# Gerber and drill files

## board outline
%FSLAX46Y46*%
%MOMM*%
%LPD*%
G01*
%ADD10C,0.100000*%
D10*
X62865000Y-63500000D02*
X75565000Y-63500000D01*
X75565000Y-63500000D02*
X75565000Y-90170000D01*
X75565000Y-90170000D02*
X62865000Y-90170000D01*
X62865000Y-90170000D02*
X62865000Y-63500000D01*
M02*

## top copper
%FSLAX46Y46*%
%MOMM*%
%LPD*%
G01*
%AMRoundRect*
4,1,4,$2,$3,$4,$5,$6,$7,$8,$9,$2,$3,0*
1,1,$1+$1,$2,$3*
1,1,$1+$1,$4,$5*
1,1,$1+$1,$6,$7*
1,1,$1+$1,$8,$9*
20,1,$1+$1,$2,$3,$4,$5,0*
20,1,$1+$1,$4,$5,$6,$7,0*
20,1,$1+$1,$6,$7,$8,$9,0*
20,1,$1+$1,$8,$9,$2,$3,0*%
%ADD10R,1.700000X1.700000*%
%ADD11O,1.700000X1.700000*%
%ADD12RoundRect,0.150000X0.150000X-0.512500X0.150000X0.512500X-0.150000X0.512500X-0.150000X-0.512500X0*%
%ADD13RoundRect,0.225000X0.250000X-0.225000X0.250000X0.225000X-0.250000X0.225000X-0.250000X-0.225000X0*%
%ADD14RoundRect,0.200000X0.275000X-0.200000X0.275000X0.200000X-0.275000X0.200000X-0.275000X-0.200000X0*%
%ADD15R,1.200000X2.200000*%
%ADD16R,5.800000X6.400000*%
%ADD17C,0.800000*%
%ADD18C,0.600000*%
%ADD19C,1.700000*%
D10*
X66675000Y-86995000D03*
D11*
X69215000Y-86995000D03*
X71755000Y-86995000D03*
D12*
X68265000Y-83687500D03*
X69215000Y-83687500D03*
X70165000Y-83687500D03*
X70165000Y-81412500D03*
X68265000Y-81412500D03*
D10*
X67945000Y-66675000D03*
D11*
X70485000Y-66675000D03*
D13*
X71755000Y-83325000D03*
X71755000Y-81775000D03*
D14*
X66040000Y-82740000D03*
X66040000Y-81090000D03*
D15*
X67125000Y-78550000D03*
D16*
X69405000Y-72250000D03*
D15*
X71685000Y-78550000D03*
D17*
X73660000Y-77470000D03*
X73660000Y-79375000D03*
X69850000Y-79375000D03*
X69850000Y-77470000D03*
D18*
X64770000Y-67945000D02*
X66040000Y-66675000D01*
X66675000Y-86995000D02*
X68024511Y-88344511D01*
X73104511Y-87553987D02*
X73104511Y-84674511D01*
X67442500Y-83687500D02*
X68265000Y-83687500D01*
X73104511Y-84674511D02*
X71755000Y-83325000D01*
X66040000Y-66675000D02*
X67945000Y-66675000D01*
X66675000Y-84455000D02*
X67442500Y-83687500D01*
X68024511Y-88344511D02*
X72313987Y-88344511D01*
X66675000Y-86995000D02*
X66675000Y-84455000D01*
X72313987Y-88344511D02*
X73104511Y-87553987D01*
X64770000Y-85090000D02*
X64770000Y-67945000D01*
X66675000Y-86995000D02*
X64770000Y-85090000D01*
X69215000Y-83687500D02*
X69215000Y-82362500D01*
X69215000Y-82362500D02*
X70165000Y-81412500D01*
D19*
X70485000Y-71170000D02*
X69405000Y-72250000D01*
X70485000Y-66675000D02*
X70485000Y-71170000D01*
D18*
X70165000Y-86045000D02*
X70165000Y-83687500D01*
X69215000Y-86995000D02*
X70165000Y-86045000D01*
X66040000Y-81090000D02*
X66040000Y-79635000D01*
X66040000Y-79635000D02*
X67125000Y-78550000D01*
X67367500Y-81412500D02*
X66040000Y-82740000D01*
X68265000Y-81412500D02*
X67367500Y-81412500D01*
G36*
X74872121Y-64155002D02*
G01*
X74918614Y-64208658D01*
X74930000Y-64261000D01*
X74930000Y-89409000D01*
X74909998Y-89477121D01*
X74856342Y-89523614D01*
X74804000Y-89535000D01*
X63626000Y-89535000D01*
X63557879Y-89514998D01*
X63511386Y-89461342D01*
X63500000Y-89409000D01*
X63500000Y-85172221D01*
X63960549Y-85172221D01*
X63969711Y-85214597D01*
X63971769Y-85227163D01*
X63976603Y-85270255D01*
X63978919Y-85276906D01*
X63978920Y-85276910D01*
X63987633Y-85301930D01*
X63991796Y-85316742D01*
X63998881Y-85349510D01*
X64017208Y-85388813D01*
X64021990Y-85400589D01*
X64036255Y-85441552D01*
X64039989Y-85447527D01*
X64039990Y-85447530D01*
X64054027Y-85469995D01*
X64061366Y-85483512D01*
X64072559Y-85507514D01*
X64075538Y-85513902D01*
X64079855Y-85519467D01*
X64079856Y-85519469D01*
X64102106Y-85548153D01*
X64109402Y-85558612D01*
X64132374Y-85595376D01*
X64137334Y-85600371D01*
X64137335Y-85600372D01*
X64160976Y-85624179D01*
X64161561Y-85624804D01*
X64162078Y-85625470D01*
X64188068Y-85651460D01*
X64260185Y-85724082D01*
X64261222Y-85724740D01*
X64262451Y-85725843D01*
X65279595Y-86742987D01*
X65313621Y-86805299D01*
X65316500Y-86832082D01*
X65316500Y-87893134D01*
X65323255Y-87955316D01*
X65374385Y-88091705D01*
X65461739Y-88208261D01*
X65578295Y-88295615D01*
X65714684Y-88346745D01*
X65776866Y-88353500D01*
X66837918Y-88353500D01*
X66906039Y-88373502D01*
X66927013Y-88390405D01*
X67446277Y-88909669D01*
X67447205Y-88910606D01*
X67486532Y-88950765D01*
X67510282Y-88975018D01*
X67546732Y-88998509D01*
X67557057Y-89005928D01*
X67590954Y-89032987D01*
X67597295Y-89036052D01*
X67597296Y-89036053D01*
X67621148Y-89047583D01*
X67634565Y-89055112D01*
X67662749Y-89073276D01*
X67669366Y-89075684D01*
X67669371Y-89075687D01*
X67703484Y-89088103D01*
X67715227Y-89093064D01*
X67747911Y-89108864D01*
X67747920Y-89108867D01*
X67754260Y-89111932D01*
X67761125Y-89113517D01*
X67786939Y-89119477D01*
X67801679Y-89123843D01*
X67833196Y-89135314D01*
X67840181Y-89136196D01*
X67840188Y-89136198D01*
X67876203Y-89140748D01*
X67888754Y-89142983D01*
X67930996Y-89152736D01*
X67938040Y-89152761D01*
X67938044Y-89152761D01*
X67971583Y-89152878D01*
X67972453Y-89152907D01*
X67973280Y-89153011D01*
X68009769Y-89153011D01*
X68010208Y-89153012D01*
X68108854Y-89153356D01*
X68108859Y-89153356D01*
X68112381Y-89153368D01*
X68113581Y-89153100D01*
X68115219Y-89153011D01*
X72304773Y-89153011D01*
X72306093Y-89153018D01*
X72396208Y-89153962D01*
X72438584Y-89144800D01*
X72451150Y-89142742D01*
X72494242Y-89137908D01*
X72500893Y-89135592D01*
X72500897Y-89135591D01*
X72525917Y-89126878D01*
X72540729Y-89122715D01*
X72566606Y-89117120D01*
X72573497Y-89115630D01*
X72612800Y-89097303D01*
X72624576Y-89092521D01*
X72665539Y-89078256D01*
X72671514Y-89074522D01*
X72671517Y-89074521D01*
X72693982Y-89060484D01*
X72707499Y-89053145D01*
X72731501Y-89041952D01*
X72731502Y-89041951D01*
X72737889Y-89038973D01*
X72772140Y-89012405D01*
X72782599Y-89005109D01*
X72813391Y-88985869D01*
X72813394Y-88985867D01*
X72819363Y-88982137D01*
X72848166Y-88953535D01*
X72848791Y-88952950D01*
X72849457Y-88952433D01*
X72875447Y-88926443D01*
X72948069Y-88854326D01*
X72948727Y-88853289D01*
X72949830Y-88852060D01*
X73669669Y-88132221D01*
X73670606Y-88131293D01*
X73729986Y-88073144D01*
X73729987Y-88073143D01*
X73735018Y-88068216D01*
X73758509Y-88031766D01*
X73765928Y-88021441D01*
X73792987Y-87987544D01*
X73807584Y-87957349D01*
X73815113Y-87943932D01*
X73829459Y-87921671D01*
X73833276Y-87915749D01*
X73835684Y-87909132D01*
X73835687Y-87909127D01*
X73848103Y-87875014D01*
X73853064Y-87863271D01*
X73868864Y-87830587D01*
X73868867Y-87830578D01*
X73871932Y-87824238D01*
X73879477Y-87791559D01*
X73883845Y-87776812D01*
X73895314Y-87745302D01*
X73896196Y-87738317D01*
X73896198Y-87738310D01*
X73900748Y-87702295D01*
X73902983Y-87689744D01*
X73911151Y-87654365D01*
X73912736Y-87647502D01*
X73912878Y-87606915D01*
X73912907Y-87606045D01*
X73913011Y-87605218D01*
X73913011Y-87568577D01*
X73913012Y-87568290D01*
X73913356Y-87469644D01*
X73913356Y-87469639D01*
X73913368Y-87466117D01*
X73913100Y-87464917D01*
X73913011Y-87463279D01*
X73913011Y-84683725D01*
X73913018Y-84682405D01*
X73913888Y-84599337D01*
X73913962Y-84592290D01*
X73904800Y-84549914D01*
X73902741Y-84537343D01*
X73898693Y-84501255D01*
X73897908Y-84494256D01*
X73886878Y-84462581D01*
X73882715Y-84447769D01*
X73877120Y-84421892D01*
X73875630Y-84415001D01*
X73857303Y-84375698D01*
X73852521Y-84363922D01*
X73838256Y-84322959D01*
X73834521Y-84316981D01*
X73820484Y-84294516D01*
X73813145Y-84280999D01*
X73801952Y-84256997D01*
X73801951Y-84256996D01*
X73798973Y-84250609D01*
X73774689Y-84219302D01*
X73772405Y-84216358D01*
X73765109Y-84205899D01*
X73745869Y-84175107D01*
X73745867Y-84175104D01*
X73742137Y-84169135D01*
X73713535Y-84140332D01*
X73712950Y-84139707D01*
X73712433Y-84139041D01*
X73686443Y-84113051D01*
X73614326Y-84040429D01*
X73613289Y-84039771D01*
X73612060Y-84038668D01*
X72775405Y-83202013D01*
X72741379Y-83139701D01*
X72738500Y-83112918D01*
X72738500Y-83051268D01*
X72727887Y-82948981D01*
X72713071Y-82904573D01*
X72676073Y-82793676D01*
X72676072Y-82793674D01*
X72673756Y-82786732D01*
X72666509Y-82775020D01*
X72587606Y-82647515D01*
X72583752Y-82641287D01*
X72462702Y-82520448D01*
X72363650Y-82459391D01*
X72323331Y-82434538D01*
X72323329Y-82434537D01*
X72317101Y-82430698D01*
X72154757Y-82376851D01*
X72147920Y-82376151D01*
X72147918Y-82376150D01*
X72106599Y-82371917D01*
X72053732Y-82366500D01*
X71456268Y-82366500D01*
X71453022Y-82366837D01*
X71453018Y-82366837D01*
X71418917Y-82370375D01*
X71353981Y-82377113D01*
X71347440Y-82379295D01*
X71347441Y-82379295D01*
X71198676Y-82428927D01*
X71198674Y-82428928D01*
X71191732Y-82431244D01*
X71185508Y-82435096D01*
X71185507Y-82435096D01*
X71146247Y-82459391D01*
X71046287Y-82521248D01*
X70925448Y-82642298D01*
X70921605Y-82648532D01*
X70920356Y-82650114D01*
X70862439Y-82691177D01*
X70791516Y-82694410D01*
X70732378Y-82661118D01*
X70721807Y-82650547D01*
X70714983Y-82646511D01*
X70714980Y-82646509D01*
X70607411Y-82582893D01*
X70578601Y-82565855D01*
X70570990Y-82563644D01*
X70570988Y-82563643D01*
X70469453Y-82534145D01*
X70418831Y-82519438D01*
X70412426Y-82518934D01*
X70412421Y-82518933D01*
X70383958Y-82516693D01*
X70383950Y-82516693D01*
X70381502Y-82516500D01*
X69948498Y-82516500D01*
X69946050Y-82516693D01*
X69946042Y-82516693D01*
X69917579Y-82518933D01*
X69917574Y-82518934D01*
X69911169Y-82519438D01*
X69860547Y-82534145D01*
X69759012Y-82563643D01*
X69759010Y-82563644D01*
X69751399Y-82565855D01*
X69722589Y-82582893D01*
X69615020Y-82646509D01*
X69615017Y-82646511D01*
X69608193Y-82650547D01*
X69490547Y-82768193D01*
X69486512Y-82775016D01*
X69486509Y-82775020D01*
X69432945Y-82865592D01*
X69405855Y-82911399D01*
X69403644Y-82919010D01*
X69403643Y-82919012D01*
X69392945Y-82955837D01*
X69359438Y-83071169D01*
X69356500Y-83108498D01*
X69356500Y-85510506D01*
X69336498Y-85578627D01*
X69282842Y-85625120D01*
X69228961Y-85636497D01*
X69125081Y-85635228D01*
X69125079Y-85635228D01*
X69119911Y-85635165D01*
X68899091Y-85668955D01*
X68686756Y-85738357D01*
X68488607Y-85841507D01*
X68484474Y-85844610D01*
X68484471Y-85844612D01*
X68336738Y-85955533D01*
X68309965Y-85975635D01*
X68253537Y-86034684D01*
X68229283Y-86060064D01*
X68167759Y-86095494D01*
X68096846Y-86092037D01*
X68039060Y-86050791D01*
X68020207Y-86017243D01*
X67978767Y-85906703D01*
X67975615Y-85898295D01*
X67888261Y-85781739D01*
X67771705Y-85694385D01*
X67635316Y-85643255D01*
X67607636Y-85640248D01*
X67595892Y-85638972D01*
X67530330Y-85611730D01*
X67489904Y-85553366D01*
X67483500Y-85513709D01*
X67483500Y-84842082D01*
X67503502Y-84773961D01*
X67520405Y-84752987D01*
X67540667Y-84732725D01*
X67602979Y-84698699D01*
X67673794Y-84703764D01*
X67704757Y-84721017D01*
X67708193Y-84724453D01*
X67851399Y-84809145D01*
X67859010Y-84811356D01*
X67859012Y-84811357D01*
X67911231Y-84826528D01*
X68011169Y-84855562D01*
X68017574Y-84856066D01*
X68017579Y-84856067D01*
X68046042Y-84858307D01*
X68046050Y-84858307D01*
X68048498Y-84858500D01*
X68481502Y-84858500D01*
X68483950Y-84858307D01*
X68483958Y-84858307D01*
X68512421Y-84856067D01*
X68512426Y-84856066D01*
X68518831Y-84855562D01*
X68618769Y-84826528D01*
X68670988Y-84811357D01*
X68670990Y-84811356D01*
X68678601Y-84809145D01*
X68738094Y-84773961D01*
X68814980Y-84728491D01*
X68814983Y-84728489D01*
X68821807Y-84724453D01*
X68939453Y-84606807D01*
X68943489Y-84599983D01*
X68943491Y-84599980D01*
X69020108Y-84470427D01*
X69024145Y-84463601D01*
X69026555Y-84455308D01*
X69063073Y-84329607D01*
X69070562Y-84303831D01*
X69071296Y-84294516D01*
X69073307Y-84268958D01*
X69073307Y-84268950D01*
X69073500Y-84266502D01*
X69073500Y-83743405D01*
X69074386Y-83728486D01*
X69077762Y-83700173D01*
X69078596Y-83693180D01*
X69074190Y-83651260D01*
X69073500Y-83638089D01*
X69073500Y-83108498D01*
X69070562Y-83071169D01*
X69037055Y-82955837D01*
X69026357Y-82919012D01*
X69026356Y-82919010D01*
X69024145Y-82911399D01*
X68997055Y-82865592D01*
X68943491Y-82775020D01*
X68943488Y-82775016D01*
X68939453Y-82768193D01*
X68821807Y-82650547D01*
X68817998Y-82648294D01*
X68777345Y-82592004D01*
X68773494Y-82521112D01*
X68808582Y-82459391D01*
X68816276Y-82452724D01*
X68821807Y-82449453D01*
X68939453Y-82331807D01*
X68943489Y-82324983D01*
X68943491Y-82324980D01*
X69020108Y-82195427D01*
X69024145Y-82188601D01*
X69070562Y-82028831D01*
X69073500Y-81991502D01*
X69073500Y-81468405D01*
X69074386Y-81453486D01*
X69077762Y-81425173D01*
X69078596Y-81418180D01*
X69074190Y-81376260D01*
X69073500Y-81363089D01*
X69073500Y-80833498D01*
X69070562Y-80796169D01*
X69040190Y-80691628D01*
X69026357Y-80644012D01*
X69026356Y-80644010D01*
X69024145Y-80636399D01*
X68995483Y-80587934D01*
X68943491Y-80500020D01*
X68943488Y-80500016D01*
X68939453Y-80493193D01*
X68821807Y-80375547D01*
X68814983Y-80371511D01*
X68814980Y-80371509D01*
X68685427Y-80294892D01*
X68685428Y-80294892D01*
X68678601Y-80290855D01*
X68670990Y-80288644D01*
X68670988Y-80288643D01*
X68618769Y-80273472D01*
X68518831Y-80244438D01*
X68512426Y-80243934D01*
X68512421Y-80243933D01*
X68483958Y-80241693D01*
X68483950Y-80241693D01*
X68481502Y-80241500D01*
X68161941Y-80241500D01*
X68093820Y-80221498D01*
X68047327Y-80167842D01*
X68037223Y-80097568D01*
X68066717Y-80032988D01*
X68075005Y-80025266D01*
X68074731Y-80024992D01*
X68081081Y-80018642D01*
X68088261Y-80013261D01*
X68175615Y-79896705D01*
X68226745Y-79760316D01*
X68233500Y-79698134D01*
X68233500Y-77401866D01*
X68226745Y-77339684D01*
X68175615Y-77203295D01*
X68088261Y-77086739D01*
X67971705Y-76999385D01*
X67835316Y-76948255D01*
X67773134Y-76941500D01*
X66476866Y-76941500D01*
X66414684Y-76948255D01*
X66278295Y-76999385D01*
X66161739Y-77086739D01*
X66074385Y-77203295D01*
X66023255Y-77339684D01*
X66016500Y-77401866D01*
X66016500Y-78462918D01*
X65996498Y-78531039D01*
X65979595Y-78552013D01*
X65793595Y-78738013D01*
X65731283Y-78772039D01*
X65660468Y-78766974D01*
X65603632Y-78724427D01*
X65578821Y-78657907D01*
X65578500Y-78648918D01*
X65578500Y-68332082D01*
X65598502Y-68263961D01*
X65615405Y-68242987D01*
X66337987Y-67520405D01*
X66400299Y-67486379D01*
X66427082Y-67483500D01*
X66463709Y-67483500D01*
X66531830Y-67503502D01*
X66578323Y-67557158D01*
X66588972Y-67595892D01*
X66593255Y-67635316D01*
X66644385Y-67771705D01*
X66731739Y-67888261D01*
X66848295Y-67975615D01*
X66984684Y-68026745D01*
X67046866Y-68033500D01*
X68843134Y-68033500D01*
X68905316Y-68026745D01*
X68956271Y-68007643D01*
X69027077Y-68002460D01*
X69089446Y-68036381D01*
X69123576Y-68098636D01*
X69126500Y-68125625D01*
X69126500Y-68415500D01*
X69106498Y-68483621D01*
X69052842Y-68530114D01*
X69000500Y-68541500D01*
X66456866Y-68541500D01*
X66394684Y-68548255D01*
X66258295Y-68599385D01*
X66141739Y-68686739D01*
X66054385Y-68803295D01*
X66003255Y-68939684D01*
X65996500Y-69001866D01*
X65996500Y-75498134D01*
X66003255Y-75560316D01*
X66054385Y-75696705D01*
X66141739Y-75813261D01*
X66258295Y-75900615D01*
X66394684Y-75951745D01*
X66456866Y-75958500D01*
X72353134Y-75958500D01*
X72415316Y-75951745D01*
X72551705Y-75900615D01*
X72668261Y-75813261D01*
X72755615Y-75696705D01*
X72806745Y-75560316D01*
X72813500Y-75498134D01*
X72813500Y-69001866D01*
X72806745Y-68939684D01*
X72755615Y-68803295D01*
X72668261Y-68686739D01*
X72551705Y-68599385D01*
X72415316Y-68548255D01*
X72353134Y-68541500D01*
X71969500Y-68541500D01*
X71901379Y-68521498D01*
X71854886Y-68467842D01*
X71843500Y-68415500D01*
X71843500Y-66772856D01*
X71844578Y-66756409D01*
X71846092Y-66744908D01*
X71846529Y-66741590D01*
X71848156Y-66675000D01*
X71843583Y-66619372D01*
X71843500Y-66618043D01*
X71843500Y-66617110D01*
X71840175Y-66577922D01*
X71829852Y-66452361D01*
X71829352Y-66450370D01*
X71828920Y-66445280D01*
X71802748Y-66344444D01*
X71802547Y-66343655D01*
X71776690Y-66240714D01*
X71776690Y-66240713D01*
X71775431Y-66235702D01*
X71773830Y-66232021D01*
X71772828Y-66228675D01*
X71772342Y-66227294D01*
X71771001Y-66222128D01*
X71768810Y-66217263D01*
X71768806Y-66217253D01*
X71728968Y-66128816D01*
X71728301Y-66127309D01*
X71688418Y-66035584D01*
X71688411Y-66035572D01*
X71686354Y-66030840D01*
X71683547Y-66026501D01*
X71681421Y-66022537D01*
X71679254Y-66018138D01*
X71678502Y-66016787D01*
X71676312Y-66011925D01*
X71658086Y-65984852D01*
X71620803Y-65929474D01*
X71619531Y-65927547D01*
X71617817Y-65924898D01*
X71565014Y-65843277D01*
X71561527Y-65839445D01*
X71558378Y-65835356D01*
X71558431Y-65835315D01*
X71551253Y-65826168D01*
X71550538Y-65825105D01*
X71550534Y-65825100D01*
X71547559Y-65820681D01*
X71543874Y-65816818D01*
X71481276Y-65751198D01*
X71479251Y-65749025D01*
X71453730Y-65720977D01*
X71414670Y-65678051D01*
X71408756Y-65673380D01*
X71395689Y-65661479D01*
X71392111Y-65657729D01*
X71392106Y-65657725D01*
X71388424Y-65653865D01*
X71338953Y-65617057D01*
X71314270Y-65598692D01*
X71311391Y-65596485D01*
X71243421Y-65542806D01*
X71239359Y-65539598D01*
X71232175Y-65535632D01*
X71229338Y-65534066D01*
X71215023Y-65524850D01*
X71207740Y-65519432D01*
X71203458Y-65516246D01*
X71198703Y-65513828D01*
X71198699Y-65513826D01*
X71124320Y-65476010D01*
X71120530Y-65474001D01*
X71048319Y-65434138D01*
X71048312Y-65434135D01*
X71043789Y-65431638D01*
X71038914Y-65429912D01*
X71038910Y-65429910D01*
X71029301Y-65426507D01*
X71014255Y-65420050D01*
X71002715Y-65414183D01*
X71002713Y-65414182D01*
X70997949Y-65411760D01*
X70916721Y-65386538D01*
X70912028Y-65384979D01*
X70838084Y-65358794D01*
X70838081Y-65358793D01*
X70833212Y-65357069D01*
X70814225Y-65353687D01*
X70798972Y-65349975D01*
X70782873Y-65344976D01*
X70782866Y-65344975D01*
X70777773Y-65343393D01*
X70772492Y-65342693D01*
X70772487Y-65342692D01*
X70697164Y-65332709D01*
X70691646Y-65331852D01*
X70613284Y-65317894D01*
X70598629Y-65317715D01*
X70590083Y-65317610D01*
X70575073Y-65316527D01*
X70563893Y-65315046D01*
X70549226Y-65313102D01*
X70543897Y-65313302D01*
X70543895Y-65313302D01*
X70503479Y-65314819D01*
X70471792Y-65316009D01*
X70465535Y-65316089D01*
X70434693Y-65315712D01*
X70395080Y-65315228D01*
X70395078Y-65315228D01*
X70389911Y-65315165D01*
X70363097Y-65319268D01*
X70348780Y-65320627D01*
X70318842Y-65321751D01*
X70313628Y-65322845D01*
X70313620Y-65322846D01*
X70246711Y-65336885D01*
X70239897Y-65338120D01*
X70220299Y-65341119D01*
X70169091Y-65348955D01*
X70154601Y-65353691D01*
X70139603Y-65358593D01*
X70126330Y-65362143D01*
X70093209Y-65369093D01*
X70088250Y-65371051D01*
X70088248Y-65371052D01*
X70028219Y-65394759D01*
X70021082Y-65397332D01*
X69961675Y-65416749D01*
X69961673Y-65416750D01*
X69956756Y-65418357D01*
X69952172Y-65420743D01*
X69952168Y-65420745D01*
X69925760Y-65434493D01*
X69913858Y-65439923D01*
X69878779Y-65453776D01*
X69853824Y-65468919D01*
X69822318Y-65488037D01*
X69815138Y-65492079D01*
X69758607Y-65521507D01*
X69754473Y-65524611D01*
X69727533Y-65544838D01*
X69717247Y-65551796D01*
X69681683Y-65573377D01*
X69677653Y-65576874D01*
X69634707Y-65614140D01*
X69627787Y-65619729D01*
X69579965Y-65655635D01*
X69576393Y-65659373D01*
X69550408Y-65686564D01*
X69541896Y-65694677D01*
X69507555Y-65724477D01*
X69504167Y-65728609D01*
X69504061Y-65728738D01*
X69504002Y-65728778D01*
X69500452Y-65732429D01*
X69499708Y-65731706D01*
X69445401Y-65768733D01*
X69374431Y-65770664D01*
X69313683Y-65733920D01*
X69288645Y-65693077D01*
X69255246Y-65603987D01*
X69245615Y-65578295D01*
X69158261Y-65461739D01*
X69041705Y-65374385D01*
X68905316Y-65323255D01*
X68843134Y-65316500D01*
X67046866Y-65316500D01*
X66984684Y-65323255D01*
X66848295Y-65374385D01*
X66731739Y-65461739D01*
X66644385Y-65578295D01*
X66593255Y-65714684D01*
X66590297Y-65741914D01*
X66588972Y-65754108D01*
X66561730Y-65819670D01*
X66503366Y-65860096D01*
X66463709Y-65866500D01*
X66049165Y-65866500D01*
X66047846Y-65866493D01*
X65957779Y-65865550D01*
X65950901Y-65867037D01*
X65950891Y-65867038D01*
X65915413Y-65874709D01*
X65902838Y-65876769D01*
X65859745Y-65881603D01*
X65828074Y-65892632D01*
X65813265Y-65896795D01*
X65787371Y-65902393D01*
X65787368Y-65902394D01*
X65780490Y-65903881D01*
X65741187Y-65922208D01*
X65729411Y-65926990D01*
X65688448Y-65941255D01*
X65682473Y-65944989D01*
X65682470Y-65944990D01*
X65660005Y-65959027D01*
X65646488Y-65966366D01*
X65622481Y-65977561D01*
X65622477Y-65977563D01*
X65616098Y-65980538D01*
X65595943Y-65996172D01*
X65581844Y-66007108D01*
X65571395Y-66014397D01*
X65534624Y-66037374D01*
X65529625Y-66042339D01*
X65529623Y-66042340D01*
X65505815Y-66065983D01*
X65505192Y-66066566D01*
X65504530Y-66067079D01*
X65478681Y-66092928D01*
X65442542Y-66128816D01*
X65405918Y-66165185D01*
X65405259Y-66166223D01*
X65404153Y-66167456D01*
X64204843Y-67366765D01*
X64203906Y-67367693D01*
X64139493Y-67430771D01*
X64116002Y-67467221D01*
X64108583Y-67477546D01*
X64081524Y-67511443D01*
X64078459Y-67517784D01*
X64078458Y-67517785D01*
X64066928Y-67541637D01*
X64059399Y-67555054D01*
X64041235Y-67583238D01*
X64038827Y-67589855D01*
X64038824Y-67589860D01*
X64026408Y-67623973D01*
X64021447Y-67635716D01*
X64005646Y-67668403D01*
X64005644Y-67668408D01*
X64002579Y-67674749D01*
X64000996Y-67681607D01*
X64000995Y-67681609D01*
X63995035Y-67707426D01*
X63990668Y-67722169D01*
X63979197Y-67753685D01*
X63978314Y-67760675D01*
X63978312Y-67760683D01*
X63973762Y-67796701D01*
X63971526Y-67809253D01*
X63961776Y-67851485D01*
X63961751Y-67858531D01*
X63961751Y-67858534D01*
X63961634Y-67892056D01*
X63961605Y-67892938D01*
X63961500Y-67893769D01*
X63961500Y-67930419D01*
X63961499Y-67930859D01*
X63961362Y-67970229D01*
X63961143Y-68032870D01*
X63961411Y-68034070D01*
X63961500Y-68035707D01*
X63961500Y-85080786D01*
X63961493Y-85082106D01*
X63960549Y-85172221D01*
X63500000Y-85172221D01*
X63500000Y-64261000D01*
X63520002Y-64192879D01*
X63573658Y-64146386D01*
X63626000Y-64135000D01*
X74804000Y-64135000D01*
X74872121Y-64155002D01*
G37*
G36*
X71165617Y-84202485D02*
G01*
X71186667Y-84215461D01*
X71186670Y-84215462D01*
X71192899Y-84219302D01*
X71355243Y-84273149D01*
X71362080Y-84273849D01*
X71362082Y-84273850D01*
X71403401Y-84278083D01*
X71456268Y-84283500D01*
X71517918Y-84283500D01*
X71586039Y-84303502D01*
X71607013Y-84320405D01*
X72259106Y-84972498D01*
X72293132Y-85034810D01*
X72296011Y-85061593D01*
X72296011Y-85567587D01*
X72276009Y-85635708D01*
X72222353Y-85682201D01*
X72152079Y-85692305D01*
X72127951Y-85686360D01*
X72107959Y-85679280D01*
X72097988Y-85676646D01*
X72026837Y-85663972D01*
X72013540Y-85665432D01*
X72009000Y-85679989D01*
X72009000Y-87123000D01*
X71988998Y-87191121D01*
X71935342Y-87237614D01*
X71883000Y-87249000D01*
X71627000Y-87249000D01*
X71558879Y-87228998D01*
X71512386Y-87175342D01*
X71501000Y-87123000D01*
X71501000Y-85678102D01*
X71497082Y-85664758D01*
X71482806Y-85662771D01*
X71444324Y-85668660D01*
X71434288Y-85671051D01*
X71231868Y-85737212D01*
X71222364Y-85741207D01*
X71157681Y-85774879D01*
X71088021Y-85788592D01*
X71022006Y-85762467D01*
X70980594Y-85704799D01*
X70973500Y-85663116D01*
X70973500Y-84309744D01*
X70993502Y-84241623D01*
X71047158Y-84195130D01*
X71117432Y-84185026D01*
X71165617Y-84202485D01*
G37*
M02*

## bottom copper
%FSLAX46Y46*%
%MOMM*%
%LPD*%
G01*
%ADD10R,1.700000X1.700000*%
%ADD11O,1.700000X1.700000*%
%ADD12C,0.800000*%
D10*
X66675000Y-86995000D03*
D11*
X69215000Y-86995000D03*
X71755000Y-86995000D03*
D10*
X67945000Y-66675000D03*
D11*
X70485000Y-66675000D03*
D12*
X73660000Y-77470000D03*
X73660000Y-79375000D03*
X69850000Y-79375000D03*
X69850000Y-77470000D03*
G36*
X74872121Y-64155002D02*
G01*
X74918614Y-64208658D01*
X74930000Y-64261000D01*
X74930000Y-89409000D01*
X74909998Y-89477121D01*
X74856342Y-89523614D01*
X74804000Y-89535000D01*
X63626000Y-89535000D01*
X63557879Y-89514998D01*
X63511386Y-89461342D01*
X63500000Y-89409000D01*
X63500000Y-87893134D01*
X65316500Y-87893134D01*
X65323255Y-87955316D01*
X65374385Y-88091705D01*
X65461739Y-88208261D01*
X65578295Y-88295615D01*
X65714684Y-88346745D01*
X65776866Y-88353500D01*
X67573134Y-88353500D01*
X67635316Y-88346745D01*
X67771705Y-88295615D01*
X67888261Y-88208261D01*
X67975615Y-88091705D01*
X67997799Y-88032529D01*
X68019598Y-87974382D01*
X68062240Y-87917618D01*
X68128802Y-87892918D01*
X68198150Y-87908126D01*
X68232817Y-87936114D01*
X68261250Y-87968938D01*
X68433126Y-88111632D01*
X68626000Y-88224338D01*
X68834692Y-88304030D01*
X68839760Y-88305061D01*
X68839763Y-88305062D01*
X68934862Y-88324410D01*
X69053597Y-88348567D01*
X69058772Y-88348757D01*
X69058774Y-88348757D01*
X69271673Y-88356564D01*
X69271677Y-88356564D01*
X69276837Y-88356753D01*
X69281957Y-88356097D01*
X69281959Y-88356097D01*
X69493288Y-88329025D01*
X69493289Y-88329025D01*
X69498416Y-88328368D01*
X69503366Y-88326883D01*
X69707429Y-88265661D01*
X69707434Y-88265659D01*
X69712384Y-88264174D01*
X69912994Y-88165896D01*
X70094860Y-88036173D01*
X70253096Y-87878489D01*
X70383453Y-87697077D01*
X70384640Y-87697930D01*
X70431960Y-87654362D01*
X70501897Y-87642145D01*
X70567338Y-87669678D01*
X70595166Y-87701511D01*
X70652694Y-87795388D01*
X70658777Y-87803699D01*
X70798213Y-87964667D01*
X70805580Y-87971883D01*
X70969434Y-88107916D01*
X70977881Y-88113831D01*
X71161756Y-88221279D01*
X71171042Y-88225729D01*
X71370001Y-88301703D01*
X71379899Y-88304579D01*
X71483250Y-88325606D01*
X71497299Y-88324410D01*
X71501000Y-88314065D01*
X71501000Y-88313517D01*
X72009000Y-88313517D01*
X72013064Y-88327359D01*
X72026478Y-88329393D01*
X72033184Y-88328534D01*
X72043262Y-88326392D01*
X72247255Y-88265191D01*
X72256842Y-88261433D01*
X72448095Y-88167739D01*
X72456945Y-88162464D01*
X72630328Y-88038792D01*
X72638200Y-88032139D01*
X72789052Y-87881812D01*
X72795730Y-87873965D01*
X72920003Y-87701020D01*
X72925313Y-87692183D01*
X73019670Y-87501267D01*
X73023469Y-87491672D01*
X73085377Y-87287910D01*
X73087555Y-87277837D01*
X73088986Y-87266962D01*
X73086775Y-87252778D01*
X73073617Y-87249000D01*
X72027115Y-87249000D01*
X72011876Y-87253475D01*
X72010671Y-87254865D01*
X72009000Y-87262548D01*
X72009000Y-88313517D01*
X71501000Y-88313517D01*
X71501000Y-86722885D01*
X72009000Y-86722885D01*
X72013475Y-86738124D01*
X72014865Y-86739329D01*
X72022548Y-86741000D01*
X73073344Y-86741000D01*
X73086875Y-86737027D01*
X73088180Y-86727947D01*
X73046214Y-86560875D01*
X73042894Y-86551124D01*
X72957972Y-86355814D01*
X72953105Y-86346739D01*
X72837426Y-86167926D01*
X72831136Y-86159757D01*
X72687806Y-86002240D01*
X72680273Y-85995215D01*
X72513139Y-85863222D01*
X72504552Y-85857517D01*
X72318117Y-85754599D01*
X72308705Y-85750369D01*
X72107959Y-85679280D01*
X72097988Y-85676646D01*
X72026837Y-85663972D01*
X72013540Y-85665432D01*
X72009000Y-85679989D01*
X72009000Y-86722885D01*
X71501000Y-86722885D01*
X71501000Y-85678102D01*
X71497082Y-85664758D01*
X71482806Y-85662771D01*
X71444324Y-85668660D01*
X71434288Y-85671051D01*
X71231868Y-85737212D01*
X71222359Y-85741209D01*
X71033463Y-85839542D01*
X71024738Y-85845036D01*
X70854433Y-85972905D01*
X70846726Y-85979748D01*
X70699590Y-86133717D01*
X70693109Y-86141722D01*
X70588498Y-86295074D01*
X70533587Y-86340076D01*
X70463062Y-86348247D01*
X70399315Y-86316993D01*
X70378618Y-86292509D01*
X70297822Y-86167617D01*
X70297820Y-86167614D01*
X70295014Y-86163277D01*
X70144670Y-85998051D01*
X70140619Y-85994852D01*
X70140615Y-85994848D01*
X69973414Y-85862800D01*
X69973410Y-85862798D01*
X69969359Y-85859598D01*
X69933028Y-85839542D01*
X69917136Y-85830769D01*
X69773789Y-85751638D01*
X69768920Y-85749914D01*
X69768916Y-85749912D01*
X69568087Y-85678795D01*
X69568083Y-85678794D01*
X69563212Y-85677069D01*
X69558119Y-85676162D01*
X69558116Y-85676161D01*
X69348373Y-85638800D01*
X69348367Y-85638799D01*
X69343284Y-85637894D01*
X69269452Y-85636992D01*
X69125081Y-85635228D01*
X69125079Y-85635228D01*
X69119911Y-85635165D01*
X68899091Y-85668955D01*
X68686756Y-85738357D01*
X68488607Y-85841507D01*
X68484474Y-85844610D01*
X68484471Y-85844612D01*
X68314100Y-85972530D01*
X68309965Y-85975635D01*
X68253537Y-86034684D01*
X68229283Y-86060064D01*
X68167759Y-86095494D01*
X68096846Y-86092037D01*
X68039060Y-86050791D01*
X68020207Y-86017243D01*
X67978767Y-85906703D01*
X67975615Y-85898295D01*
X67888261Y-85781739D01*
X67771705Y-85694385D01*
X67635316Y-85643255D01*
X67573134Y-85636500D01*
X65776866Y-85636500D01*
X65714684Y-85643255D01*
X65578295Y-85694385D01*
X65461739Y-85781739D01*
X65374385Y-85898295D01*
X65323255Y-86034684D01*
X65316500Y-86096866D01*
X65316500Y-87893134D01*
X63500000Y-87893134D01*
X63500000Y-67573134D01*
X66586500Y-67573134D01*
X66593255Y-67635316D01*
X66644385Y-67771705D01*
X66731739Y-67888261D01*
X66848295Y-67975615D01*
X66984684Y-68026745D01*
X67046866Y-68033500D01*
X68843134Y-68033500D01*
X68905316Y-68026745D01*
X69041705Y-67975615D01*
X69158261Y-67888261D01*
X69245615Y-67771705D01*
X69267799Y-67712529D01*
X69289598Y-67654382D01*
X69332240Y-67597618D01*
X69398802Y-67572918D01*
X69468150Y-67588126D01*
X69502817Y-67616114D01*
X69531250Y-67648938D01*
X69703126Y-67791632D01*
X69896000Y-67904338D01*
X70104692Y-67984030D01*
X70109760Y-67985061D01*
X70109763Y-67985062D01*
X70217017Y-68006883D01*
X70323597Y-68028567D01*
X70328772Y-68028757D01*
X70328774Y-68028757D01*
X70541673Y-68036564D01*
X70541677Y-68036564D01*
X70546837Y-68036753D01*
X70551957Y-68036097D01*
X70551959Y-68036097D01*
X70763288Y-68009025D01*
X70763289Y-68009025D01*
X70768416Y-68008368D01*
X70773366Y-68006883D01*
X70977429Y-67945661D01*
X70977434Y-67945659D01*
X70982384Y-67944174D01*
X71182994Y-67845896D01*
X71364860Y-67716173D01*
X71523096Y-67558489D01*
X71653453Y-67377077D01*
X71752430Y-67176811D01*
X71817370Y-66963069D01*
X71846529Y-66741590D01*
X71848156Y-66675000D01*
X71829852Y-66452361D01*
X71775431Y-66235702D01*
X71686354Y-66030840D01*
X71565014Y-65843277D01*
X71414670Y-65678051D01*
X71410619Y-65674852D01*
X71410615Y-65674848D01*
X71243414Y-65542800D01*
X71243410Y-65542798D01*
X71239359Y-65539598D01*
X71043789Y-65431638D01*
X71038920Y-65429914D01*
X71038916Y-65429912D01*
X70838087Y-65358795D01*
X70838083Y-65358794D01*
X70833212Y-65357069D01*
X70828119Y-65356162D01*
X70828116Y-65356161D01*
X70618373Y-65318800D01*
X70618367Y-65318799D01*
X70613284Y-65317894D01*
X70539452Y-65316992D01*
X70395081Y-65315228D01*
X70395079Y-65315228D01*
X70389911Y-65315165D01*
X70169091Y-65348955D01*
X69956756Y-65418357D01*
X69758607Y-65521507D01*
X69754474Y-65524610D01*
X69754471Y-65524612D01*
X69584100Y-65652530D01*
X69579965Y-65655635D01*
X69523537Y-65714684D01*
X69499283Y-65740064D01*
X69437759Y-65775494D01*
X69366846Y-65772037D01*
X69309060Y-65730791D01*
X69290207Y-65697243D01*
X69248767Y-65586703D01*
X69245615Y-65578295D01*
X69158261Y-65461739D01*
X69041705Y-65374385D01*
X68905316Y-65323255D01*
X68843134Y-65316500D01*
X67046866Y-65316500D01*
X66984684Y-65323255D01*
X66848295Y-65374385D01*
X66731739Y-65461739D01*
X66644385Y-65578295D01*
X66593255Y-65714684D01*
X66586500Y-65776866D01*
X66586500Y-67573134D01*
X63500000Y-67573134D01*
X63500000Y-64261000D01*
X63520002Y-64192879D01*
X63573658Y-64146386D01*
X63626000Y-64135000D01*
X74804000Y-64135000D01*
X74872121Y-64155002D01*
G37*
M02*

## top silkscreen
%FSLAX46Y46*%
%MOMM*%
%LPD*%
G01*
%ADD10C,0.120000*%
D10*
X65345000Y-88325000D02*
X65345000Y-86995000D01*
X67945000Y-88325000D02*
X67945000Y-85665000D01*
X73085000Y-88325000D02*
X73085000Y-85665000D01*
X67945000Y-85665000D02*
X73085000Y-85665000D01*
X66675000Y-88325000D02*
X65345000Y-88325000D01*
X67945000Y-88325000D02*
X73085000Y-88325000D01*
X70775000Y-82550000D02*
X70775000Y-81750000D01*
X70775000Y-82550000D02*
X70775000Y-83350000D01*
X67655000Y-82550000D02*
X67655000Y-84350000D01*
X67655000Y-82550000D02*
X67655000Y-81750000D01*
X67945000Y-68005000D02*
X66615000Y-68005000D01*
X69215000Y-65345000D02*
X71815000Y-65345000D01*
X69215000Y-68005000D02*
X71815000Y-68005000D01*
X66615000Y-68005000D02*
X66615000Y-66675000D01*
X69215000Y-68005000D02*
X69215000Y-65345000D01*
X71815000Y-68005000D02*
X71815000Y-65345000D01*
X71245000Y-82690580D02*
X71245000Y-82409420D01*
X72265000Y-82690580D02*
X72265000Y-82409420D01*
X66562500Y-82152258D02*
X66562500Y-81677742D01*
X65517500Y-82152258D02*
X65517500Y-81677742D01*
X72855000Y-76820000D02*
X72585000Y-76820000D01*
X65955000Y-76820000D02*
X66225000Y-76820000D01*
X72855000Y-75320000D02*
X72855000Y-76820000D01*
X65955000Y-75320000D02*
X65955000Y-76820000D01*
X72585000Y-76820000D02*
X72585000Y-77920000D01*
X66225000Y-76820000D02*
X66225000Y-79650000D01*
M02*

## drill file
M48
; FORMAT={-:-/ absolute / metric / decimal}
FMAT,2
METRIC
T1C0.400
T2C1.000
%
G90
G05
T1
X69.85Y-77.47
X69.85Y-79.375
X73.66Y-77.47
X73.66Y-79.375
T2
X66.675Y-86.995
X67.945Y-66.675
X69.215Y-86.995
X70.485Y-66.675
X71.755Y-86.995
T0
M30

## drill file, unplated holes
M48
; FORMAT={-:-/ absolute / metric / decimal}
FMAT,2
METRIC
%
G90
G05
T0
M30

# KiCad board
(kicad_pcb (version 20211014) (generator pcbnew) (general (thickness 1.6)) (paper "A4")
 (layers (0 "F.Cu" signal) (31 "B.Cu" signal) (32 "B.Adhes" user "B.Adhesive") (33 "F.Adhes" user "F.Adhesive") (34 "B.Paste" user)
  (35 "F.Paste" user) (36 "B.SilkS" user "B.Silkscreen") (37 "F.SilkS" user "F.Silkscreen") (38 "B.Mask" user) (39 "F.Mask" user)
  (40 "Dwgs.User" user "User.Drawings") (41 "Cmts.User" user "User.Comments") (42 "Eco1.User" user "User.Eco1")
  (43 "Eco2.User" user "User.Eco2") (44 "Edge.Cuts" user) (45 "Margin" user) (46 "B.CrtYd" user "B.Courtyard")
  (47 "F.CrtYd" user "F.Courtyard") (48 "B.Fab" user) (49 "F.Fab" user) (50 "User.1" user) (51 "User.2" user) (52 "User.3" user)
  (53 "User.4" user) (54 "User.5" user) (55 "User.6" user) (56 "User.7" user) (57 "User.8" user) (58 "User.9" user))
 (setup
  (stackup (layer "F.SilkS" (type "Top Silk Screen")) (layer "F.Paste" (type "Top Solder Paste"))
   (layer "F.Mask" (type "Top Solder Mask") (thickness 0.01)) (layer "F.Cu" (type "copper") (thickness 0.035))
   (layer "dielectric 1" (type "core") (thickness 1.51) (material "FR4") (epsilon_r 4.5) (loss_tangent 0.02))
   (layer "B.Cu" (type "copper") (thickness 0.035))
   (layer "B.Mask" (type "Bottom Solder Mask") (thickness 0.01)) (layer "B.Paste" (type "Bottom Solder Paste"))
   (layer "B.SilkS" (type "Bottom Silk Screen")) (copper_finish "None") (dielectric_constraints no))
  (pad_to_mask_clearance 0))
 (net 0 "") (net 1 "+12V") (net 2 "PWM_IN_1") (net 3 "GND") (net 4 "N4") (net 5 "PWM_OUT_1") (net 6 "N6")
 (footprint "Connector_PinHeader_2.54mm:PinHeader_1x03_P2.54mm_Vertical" (layer "F.Cu") (at 66.675 86.995 90)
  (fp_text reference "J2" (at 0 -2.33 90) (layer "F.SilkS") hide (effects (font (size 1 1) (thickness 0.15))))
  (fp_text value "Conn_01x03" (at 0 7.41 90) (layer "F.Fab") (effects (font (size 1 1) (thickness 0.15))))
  (fp_line (start -1.33 -1.33) (end 0 -1.33) (layer "F.SilkS") (width 0.12))
  (fp_line (start -1.33 1.27) (end 1.33 1.27) (layer "F.SilkS") (width 0.12))
  (fp_line (start -1.33 6.41) (end 1.33 6.41) (layer "F.SilkS") (width 0.12))
  (fp_line (start 1.33 1.27) (end 1.33 6.41) (layer "F.SilkS") (width 0.12))
  (fp_line (start -1.33 0) (end -1.33 -1.33) (layer "F.SilkS") (width 0.12))
  (fp_line (start -1.33 1.27) (end -1.33 6.41) (layer "F.SilkS") (width 0.12))
  (pad "1" thru_hole rect (at 0 0 90) (size 1.7 1.7) (drill 1) (layers *.Cu *.Mask) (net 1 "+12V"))
  (pad "2" thru_hole oval (at 0 2.54 90) (size 1.7 1.7) (drill 1) (layers *.Cu *.Mask) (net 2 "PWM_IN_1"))
  (pad "3" thru_hole oval (at 0 5.08 90) (size 1.7 1.7) (drill 1) (layers *.Cu *.Mask) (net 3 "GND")))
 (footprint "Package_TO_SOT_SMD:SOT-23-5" (layer "F.Cu") (at 69.215 82.55 90)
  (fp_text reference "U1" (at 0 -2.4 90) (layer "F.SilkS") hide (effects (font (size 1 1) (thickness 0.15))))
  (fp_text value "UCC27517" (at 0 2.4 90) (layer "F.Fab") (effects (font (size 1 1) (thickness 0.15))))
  (fp_line (start 0 1.56) (end 0.8 1.56) (layer "F.SilkS") (width 0.12))
  (fp_line (start 0 1.56) (end -0.8 1.56) (layer "F.SilkS") (width 0.12))
  (fp_line (start 0 -1.56) (end -1.8 -1.56) (layer "F.SilkS") (width 0.12))
  (fp_line (start 0 -1.56) (end 0.8 -1.56) (layer "F.SilkS") (width 0.12))
  (pad "1" smd roundrect (at -1.1375 -0.95 90) (size 1.325 0.6) (layers "F.Cu" "F.Paste" "F.Mask") (roundrect_rratio 0.25) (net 1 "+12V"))
  (pad "2" smd roundrect (at -1.1375 0 90) (size 1.325 0.6) (layers "F.Cu" "F.Paste" "F.Mask") (roundrect_rratio 0.25) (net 3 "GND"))
  (pad "3" smd roundrect (at -1.1375 0.95 90) (size 1.325 0.6) (layers "F.Cu" "F.Paste" "F.Mask") (roundrect_rratio 0.25) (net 2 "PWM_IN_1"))
  (pad "4" smd roundrect (at 1.1375 0.95 90) (size 1.325 0.6) (layers "F.Cu" "F.Paste" "F.Mask") (roundrect_rratio 0.25) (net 3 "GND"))
  (pad "5" smd roundrect (at 1.1375 -0.95 90) (size 1.325 0.6) (layers "F.Cu" "F.Paste" "F.Mask") (roundrect_rratio 0.25) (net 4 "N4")))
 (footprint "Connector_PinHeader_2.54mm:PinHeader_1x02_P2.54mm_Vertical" (layer "F.Cu") (at 67.945 66.675 90)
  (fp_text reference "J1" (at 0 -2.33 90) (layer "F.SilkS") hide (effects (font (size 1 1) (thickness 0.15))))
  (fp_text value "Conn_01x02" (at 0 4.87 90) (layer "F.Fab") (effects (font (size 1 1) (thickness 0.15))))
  (fp_line (start -1.33 0) (end -1.33 -1.33) (layer "F.SilkS") (width 0.12))
  (fp_line (start 1.33 1.27) (end 1.33 3.87) (layer "F.SilkS") (width 0.12))
  (fp_line (start -1.33 1.27) (end -1.33 3.87) (layer "F.SilkS") (width 0.12))
  (fp_line (start -1.33 -1.33) (end 0 -1.33) (layer "F.SilkS") (width 0.12))
  (fp_line (start -1.33 1.27) (end 1.33 1.27) (layer "F.SilkS") (width 0.12))
  (fp_line (start -1.33 3.87) (end 1.33 3.87) (layer "F.SilkS") (width 0.12))
  (pad "1" thru_hole rect (at 0 0 90) (size 1.7 1.7) (drill 1) (layers *.Cu *.Mask) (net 1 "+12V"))
  (pad "2" thru_hole oval (at 0 2.54 90) (size 1.7 1.7) (drill 1) (layers *.Cu *.Mask) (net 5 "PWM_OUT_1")))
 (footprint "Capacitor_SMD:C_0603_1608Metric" (layer "F.Cu") (at 71.755 82.55 90)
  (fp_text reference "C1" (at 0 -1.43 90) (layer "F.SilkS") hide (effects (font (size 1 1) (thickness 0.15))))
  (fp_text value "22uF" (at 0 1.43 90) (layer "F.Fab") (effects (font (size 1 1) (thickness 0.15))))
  (fp_line (start -0.14058 -0.51) (end 0.14058 -0.51) (layer "F.SilkS") (width 0.12))
  (fp_line (start -0.14058 0.51) (end 0.14058 0.51) (layer "F.SilkS") (width 0.12))
  (pad "1" smd roundrect (at -0.775 0 90) (size 0.9 0.95) (layers "F.Cu" "F.Paste" "F.Mask") (roundrect_rratio 0.25) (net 1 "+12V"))
  (pad "2" smd roundrect (at 0.775 0 90) (size 0.9 0.95) (layers "F.Cu" "F.Paste" "F.Mask") (roundrect_rratio 0.25) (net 3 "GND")))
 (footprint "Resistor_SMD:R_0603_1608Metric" (layer "F.Cu") (at 66.04 81.915 90)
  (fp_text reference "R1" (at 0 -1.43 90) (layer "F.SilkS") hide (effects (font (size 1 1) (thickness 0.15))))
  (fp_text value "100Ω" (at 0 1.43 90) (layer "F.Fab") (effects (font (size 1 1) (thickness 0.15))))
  (fp_line (start -0.237258 0.5225) (end 0.237258 0.5225) (layer "F.SilkS") (width 0.12))
  (fp_line (start -0.237258 -0.5225) (end 0.237258 -0.5225) (layer "F.SilkS") (width 0.12))
  (pad "1" smd roundrect (at -0.825 0 90) (size 0.8 0.95) (layers "F.Cu" "F.Paste" "F.Mask") (roundrect_rratio 0.25) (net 4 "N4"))
  (pad "2" smd roundrect (at 0.825 0 90) (size 0.8 0.95) (layers "F.Cu" "F.Paste" "F.Mask") (roundrect_rratio 0.25) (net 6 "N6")))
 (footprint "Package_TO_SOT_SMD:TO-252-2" (layer "F.Cu") (at 69.405 74.35 90)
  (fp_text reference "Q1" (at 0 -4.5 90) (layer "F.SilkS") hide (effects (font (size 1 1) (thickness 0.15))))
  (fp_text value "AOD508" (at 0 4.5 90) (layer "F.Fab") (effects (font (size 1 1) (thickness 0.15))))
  (fp_line (start -2.47 3.45) (end -2.47 3.18) (layer "F.SilkS") (width 0.12))
  (fp_line (start -2.47 -3.45) (end -2.47 -3.18) (layer "F.SilkS") (width 0.12))
  (fp_line (start -0.97 3.45) (end -2.47 3.45) (layer "F.SilkS") (width 0.12))
  (fp_line (start -0.97 -3.45) (end -2.47 -3.45) (layer "F.SilkS") (width 0.12))
  (fp_line (start -2.47 3.18) (end -3.57 3.18) (layer "F.SilkS") (width 0.12))
  (fp_line (start -2.47 -3.18) (end -5.3 -3.18) (layer "F.SilkS") (width 0.12))
  (pad "" smd rect (at 3.775 -1.525 90) (size 3.05 2.75) (layers "F.Paste"))
  (pad "" smd rect (at 0.425 1.525 90) (size 3.05 2.75) (layers "F.Paste"))
  (pad "" smd rect (at 3.775 1.525 90) (size 3.05 2.75) (layers "F.Paste"))
  (pad "" smd rect (at 0.425 -1.525 90) (size 3.05 2.75) (layers "F.Paste"))
  (pad "1" smd rect (at -4.2 -2.28 90) (size 2.2 1.2) (layers "F.Cu" "F.Paste" "F.Mask") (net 6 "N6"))
  (pad "2" smd rect (at 2.1 0 90) (size 6.4 5.8) (layers "F.Cu" "F.Mask") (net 5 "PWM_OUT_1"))
  (pad "3" smd rect (at -4.2 2.28 90) (size 2.2 1.2) (layers "F.Cu" "F.Paste" "F.Mask") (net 3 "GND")))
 (gr_rect (start 62.865 63.5) (end 75.565 90.17) (layer "Edge.Cuts") (width 0.1) (fill none))
 (segment (start 64.77 67.945) (end 66.04 66.675) (width 0.6) (layer "F.Cu") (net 1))
 (segment (start 66.675 86.995) (end 68.024511 88.344511) (width 0.6) (layer "F.Cu") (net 1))
 (segment (start 73.104511 87.553987) (end 73.104511 84.674511) (width 0.6) (layer "F.Cu") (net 1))
 (segment (start 67.4425 83.6875) (end 68.265 83.6875) (width 0.6) (layer "F.Cu") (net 1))
 (segment (start 73.104511 84.674511) (end 71.755 83.325) (width 0.6) (layer "F.Cu") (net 1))
 (segment (start 66.04 66.675) (end 67.945 66.675) (width 0.6) (layer "F.Cu") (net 1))
 (segment (start 66.675 84.455) (end 67.4425 83.6875) (width 0.6) (layer "F.Cu") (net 1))
 (segment (start 68.024511 88.344511) (end 72.313987 88.344511) (width 0.6) (layer "F.Cu") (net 1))
 (segment (start 66.675 86.995) (end 66.675 84.455) (width 0.6) (layer "F.Cu") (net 1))
 (segment (start 72.313987 88.344511) (end 73.104511 87.553987) (width 0.6) (layer "F.Cu") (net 1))
 (segment (start 64.77 85.09) (end 64.77 67.945) (width 0.6) (layer "F.Cu") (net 1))
 (segment (start 66.675 86.995) (end 64.77 85.09) (width 0.6) (layer "F.Cu") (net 1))
 (segment (start 69.215 83.6875) (end 69.215 82.3625) (width 0.6) (layer "F.Cu") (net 3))
 (segment (start 69.215 82.3625) (end 70.165 81.4125) (width 0.6) (layer "F.Cu") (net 3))
 (via (at 73.66 77.47) (size 0.8) (drill 0.4) (layers "F.Cu" "B.Cu") (free) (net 3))
 (via (at 73.66 79.375) (size 0.8) (drill 0.4) (layers "F.Cu" "B.Cu") (free) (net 3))
 (via (at 69.85 79.375) (size 0.8) (drill 0.4) (layers "F.Cu" "B.Cu") (free) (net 3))
 (via (at 69.85 77.47) (size 0.8) (drill 0.4) (layers "F.Cu" "B.Cu") (free) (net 3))
 (segment (start 70.485 71.17) (end 69.405 72.25) (width 1.7) (layer "F.Cu") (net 5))
 (segment (start 70.485 66.675) (end 70.485 71.17) (width 1.7) (layer "F.Cu") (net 5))
 (segment (start 70.165 86.045) (end 70.165 83.6875) (width 0.6) (layer "F.Cu") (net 2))
 (segment (start 69.215 86.995) (end 70.165 86.045) (width 0.6) (layer "F.Cu") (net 2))
 (segment (start 66.04 81.09) (end 66.04 79.635) (width 0.6) (layer "F.Cu") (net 6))
 (segment (start 66.04 79.635) (end 67.125 78.55) (width 0.6) (layer "F.Cu") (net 6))
 (segment (start 67.3675 81.4125) (end 66.04 82.74) (width 0.6) (layer "F.Cu") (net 4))
 (segment (start 68.265 81.4125) (end 67.3675 81.4125) (width 0.6) (layer "F.Cu") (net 4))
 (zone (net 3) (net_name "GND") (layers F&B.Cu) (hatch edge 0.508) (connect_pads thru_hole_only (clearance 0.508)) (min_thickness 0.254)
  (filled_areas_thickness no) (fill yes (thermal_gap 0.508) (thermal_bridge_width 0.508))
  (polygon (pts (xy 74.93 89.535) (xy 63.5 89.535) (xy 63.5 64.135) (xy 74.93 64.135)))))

